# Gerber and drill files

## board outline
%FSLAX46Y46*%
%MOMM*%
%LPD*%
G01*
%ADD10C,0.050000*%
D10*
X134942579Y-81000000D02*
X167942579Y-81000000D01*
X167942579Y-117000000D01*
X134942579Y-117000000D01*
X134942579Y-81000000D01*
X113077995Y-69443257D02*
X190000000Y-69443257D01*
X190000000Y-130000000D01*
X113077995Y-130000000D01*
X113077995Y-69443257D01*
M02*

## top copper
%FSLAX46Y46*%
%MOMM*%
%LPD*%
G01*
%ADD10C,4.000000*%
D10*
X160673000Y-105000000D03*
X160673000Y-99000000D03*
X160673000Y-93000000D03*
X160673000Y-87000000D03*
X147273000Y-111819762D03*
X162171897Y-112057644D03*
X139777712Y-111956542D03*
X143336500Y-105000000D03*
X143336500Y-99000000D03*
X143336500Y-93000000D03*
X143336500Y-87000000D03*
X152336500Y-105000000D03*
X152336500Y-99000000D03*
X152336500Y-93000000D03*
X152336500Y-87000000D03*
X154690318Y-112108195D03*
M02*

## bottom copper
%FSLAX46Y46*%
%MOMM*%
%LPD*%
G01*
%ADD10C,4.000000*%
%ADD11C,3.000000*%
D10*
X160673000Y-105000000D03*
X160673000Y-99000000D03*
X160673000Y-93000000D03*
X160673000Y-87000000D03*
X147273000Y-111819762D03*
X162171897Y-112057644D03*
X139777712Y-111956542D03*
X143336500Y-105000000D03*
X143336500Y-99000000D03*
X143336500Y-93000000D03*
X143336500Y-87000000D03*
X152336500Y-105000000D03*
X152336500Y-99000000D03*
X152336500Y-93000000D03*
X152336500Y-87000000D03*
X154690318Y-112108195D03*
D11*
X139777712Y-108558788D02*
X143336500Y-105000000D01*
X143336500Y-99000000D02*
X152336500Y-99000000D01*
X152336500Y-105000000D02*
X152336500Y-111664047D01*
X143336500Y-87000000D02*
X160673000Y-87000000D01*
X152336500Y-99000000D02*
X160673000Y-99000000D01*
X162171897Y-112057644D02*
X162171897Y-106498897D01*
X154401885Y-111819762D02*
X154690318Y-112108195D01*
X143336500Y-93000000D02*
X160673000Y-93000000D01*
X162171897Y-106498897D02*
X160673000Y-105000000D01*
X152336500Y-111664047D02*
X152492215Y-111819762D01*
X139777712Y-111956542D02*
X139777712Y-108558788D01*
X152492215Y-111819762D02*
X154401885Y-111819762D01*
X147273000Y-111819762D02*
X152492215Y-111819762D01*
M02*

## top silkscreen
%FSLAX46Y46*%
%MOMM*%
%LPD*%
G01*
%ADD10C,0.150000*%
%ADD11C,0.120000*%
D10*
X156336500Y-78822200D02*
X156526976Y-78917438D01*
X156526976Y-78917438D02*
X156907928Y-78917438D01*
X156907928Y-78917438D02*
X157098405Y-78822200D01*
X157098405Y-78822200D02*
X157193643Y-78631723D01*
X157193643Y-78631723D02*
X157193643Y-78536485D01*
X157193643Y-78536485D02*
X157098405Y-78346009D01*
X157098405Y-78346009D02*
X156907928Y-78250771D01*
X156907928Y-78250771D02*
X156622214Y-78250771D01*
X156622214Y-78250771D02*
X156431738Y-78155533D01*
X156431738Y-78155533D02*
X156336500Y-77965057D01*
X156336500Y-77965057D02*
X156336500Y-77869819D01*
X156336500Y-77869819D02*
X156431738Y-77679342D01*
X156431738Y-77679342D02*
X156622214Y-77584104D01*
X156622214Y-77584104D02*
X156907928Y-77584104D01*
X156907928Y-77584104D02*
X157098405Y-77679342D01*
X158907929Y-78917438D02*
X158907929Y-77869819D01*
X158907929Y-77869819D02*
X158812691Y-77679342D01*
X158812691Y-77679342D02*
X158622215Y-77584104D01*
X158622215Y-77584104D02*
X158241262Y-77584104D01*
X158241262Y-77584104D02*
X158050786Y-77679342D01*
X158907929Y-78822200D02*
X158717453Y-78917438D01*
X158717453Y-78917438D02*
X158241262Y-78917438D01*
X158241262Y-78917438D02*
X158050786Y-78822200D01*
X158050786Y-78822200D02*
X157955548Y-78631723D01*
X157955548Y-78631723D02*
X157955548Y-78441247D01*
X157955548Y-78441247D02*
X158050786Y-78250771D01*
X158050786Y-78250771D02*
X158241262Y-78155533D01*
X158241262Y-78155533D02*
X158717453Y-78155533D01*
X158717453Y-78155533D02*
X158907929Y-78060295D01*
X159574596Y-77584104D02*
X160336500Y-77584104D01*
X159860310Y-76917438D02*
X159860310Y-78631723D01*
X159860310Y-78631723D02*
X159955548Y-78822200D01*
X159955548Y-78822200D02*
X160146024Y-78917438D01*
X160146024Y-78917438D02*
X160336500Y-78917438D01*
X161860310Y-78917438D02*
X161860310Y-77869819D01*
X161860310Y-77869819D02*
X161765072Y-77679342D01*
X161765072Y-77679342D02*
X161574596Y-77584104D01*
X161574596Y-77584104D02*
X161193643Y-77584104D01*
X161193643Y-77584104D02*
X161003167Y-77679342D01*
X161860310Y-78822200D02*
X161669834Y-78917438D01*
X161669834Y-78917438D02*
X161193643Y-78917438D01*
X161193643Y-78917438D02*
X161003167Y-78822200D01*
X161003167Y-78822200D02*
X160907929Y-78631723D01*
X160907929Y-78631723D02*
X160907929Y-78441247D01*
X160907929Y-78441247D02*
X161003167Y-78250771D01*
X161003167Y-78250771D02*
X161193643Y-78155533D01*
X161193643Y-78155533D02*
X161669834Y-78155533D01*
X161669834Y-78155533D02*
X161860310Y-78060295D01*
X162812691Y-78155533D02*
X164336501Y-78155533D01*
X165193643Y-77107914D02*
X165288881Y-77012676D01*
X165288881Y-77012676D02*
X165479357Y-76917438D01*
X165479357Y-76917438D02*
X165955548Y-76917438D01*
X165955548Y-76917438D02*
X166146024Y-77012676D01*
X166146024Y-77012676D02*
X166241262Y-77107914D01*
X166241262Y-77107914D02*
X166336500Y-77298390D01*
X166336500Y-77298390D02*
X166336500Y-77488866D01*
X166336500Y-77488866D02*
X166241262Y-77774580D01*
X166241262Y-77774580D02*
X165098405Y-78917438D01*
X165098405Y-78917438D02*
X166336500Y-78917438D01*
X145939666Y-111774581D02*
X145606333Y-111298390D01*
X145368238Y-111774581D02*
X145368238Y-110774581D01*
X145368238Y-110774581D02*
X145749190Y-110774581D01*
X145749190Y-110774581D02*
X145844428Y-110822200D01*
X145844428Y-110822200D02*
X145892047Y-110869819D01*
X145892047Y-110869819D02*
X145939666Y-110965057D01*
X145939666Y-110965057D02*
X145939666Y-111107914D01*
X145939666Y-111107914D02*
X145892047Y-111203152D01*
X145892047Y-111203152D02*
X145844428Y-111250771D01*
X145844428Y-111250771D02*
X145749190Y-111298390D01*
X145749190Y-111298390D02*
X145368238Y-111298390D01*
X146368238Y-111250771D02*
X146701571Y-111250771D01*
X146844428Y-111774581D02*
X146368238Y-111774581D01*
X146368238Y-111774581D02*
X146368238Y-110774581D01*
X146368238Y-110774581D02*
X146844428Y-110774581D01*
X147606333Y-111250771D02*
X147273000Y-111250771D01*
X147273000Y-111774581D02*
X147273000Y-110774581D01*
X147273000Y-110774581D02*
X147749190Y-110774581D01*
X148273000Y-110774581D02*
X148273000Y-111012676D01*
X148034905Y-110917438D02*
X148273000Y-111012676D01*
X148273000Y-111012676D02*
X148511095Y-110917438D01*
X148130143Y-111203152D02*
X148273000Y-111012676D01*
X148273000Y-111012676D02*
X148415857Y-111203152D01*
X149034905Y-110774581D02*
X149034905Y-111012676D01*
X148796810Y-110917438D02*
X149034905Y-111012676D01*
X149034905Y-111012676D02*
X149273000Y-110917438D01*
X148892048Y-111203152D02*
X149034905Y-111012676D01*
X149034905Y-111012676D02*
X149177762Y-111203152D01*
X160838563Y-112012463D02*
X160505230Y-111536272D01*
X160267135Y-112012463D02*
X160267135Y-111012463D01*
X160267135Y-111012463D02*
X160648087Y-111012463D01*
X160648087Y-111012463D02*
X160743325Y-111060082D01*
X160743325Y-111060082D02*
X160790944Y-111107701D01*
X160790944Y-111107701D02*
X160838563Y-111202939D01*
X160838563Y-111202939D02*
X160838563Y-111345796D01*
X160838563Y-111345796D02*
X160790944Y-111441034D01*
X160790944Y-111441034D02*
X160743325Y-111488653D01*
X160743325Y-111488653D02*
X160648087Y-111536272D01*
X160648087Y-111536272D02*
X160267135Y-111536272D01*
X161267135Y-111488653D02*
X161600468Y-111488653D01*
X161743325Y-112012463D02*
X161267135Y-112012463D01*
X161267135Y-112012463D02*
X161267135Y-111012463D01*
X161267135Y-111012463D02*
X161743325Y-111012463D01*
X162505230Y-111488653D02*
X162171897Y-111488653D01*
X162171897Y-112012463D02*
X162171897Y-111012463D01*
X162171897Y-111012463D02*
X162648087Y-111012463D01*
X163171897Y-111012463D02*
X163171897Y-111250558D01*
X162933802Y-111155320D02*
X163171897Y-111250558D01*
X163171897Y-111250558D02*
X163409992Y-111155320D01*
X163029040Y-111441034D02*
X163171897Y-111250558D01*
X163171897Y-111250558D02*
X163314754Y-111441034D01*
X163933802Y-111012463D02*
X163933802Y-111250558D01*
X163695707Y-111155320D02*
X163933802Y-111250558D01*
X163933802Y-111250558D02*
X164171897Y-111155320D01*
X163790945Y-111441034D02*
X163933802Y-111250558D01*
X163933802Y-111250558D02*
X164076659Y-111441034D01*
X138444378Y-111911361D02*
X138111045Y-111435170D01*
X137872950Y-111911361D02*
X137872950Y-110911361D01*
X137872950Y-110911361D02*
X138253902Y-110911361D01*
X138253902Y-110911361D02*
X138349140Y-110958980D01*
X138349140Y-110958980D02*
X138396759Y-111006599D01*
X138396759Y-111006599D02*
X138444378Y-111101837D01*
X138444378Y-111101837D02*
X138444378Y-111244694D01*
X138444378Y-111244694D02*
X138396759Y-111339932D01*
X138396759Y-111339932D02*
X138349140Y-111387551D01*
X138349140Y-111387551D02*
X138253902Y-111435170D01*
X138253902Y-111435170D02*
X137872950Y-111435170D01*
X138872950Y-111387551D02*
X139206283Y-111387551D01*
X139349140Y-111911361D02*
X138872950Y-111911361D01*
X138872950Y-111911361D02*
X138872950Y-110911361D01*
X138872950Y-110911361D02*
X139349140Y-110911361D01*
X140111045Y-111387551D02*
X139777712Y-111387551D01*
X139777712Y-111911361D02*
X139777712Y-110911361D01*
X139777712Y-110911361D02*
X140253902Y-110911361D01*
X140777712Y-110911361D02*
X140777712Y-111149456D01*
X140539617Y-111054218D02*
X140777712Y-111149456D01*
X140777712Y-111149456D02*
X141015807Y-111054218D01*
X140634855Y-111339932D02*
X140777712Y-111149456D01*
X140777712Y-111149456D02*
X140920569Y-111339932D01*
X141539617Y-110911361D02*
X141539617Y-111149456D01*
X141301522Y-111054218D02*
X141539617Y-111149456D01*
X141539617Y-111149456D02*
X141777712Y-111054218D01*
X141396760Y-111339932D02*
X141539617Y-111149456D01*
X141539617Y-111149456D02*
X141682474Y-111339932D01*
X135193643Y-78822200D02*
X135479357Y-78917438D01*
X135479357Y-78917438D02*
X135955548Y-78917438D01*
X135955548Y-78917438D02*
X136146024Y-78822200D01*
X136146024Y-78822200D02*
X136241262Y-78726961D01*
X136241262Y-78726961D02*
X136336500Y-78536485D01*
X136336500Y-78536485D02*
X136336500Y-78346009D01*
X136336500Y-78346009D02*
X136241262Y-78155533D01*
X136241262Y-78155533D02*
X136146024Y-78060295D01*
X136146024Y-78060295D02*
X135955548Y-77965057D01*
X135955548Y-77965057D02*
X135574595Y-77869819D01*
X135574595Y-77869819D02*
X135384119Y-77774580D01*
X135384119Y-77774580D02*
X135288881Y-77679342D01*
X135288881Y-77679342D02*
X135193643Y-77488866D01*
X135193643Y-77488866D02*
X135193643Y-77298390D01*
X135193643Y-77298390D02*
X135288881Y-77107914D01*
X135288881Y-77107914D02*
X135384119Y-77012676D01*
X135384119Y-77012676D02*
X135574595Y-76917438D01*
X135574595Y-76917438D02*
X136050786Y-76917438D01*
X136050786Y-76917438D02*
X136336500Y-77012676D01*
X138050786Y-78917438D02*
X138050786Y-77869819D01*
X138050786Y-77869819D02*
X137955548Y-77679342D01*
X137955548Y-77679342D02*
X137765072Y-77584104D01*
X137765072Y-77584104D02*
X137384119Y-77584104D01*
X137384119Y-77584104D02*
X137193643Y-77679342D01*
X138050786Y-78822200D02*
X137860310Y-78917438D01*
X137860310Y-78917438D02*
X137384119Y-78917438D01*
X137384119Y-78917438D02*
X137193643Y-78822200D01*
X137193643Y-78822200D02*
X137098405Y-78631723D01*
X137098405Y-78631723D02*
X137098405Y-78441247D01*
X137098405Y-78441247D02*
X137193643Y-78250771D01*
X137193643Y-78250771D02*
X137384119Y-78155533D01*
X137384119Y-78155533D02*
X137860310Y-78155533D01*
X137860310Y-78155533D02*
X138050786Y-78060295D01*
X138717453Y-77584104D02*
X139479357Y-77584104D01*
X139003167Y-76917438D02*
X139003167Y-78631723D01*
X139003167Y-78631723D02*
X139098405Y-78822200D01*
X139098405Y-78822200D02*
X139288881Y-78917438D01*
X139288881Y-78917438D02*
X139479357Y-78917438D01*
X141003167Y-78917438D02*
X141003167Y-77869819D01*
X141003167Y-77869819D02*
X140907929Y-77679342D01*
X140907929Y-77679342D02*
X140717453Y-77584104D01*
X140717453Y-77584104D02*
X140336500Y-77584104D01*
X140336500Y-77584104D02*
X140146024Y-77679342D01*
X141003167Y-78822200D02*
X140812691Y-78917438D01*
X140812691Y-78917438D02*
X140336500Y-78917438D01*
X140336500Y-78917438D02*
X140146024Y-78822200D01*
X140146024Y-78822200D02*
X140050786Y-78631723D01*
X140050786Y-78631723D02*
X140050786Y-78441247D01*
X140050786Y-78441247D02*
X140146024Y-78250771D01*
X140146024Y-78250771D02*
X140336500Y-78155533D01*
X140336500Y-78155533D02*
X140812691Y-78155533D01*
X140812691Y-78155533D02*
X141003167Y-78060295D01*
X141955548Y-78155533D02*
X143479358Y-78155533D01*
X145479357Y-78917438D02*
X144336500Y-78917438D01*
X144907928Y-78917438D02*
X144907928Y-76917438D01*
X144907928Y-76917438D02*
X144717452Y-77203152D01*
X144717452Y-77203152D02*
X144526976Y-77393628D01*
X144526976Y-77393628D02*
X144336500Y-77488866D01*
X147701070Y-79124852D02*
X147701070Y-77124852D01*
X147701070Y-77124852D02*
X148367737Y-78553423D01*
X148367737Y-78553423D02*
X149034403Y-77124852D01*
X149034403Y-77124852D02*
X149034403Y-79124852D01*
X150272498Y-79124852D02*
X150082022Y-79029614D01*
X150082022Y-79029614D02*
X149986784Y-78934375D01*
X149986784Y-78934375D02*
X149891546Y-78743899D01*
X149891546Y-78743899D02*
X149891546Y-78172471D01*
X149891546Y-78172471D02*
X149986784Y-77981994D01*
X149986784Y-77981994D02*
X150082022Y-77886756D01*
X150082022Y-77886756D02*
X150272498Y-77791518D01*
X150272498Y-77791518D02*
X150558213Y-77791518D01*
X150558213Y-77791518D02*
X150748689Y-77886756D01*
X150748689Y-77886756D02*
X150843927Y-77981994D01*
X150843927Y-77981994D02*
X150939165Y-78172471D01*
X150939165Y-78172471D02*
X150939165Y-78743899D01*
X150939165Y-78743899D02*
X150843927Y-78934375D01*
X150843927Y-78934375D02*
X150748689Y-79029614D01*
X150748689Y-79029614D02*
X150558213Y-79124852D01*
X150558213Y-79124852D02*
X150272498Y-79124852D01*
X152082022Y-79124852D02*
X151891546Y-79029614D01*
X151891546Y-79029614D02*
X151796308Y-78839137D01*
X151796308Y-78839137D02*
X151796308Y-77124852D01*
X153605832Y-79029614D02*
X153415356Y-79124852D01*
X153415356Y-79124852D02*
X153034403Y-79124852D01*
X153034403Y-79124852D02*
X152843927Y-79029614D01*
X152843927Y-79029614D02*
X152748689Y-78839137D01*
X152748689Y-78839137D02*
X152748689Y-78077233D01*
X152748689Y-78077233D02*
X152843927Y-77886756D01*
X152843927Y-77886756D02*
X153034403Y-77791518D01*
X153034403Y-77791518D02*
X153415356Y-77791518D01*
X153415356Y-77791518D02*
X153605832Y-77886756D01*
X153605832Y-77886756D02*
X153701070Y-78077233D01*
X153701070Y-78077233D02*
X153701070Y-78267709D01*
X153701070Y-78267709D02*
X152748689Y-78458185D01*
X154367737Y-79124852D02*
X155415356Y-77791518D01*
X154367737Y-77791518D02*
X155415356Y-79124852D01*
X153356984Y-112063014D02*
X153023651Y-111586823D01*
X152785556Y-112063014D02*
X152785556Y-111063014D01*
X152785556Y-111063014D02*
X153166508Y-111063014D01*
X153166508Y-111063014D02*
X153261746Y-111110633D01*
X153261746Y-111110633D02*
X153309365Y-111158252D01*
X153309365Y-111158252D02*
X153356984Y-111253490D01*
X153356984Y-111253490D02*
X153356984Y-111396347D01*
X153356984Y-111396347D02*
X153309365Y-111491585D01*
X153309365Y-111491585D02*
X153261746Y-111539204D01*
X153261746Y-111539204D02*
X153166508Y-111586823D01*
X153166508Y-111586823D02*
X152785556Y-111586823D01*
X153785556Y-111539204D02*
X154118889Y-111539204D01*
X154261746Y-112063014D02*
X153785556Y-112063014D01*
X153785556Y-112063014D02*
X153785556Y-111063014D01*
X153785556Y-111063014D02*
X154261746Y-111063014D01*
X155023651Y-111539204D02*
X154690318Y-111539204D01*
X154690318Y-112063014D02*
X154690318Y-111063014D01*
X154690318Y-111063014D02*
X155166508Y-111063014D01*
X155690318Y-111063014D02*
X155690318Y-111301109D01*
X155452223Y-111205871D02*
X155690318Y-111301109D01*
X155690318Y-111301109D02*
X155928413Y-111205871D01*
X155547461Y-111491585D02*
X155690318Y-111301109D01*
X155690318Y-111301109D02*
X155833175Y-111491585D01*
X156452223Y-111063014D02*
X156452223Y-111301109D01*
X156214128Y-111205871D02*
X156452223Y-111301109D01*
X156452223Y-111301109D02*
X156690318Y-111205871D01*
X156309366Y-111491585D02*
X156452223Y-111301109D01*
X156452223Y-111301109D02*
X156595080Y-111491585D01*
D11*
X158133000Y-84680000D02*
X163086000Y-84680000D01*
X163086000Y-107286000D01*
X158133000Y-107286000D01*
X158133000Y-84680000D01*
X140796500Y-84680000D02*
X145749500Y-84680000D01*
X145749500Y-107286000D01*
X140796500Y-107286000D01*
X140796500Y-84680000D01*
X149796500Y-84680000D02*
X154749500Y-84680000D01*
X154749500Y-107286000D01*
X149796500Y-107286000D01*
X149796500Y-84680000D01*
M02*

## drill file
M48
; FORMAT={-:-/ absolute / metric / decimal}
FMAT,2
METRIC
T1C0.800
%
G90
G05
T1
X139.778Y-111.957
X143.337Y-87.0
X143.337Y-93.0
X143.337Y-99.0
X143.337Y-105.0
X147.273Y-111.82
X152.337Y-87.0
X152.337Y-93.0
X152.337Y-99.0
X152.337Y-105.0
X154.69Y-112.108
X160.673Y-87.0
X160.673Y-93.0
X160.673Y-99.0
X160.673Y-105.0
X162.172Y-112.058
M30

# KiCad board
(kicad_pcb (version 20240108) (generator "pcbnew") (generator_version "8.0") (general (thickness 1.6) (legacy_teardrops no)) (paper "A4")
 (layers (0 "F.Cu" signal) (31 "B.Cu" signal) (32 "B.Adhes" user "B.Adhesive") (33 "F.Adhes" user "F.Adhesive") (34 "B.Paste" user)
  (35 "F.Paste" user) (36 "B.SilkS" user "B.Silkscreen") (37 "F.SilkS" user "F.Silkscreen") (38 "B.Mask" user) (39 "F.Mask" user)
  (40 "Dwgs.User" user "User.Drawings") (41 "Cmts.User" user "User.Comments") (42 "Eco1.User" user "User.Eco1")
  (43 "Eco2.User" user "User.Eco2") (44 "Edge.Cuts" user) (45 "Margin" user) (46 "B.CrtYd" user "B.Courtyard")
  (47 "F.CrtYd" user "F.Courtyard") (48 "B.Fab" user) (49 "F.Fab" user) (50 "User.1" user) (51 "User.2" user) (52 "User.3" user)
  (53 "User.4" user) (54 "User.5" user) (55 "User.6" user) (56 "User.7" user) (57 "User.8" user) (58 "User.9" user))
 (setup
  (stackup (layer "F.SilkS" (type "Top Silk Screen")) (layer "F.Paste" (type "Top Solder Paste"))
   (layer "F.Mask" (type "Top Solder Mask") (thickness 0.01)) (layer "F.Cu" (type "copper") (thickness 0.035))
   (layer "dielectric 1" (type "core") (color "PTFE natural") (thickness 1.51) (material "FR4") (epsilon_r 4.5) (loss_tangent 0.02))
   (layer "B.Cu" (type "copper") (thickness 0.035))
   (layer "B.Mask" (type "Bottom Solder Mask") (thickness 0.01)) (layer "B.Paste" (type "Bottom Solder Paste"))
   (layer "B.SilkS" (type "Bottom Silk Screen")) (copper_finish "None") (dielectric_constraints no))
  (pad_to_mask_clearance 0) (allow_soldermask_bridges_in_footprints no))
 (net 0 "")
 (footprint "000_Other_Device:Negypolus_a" (layer "F.Cu") (at 160.673 105)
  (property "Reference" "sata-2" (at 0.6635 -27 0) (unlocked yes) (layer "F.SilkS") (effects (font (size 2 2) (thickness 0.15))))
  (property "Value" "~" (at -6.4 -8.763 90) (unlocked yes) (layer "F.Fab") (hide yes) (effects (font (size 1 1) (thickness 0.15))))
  (fp_rect (start -2.54 -20.32) (end 2.413 2.286) (stroke (width 0.12) (type default)) (fill none) (layer "F.SilkS"))
  (pad "1" thru_hole circle (at 0 0) (size 4 4) (drill 0.8) (layers "*.Cu" "*.Mask") (remove_unused_layers no))
  (pad "2" thru_hole circle (at 0 -6) (size 4 4) (drill 0.8) (layers "*.Cu" "*.Mask") (remove_unused_layers no))
  (pad "3" thru_hole circle (at 0 -12) (size 4 4) (drill 0.8) (layers "*.Cu" "*.Mask") (remove_unused_layers no))
  (pad "4" thru_hole circle (at 0 -18) (size 4 4) (drill 0.8) (layers "*.Cu" "*.Mask") (remove_unused_layers no)))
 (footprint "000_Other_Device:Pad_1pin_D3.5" (layer "F.Cu") (at 147.273 111.819762)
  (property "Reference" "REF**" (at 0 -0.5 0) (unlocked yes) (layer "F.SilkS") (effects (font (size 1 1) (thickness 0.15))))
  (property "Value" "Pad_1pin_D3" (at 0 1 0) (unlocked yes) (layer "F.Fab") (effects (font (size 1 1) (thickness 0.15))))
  (pad "2" thru_hole circle (at 0 0) (size 4 4) (drill 0.8) (layers "*.Cu" "*.Mask") (remove_unused_layers no)))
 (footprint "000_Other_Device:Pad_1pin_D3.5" (layer "F.Cu") (at 162.171897 112.057644)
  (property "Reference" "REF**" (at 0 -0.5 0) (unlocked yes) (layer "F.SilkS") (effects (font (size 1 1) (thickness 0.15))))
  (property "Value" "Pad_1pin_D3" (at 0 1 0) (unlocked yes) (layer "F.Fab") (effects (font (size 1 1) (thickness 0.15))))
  (pad "4" thru_hole circle (at 0 0) (size 4 4) (drill 0.8) (layers "*.Cu" "*.Mask") (remove_unused_layers no)))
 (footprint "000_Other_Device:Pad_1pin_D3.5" (layer "F.Cu") (at 139.777712 111.956542)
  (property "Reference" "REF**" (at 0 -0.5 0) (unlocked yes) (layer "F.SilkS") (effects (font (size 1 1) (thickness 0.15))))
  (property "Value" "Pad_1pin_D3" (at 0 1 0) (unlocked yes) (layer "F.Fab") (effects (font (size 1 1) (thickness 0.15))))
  (pad "1" thru_hole circle (at 0 0) (size 4 4) (drill 0.8) (layers "*.Cu" "*.Mask") (remove_unused_layers no)))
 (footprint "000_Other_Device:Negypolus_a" (layer "F.Cu") (at 143.3365 105)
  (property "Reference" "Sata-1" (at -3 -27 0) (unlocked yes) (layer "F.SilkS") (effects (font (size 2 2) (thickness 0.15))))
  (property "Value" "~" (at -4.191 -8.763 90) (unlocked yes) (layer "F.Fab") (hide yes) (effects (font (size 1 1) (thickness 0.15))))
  (fp_rect (start -2.54 -20.32) (end 2.413 2.286) (stroke (width 0.12) (type default)) (fill none) (layer "F.SilkS"))
  (pad "1" thru_hole circle (at 0 0) (size 4 4) (drill 0.8) (layers "*.Cu" "*.Mask") (remove_unused_layers no))
  (pad "2" thru_hole circle (at 0 -6) (size 4 4) (drill 0.8) (layers "*.Cu" "*.Mask") (remove_unused_layers no))
  (pad "3" thru_hole circle (at 0 -12) (size 4 4) (drill 0.8) (layers "*.Cu" "*.Mask") (remove_unused_layers no))
  (pad "4" thru_hole circle (at 0 -18) (size 4 4) (drill 0.8) (layers "*.Cu" "*.Mask") (remove_unused_layers no)))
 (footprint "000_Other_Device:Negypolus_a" (layer "F.Cu") (at 152.3365 105)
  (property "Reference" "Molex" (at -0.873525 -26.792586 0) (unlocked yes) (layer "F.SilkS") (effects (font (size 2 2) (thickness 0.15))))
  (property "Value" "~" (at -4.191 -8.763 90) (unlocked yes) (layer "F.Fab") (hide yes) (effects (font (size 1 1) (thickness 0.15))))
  (fp_rect (start -2.54 -20.32) (end 2.413 2.286) (stroke (width 0.12) (type default)) (fill none) (layer "F.SilkS"))
  (pad "1" thru_hole circle (at 0 0) (size 4 4) (drill 0.8) (layers "*.Cu" "*.Mask") (remove_unused_layers no))
  (pad "2" thru_hole circle (at 0 -6) (size 4 4) (drill 0.8) (layers "*.Cu" "*.Mask") (remove_unused_layers no))
  (pad "3" thru_hole circle (at 0 -12) (size 4 4) (drill 0.8) (layers "*.Cu" "*.Mask") (remove_unused_layers no))
  (pad "4" thru_hole circle (at 0 -18) (size 4 4) (drill 0.8) (layers "*.Cu" "*.Mask") (remove_unused_layers no)))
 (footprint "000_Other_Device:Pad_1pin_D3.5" (layer "F.Cu") (at 154.690318 112.108195)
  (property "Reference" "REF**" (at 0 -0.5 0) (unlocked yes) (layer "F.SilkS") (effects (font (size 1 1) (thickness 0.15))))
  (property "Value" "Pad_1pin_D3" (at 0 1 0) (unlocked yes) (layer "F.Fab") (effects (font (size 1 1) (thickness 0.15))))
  (pad "3" thru_hole circle (at 0 0) (size 4 4) (drill 0.8) (layers "*.Cu" "*.Mask") (remove_unused_layers no)))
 (gr_rect (start 134.942579 81) (end 167.942579 117) (stroke (width 0.05) (type default)) (fill none) (layer "Edge.Cuts"))
 (gr_rect (start 113.077995 69.443257) (end 190 130) (locked yes) (stroke (width 0.05) (type default)) (fill none) (layer "Edge.Cuts"))
 (segment (start 139.777712 108.558788) (end 143.3365 105) (width 3) (layer "B.Cu") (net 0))
 (segment (start 143.3365 99) (end 152.3365 99) (width 3) (layer "B.Cu") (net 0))
 (segment (start 152.3365 105) (end 152.3365 111.664047) (width 3) (layer "B.Cu") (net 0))
 (segment (start 143.3365 87) (end 160.673 87) (width 3) (layer "B.Cu") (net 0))
 (segment (start 152.3365 99) (end 160.673 99) (width 3) (layer "B.Cu") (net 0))
 (segment (start 162.171897 112.057644) (end 162.171897 106.498897) (width 3) (layer "B.Cu") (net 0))
 (segment (start 154.401885 111.819762) (end 154.690318 112.108195) (width 3) (layer "B.Cu") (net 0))
 (segment (start 143.3365 93) (end 160.673 93) (width 3) (layer "B.Cu") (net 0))
 (segment (start 162.171897 106.498897) (end 160.673 105) (width 3) (layer "B.Cu") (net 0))
 (segment (start 152.3365 111.664047) (end 152.492215 111.819762) (width 3) (layer "B.Cu") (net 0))
 (segment (start 139.777712 111.956542) (end 139.777712 108.558788) (width 3) (layer "B.Cu") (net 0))
 (segment (start 152.492215 111.819762) (end 154.401885 111.819762) (width 3) (layer "B.Cu") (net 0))
 (segment (start 147.273 111.819762) (end 152.492215 111.819762) (width 3) (layer "B.Cu") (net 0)))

